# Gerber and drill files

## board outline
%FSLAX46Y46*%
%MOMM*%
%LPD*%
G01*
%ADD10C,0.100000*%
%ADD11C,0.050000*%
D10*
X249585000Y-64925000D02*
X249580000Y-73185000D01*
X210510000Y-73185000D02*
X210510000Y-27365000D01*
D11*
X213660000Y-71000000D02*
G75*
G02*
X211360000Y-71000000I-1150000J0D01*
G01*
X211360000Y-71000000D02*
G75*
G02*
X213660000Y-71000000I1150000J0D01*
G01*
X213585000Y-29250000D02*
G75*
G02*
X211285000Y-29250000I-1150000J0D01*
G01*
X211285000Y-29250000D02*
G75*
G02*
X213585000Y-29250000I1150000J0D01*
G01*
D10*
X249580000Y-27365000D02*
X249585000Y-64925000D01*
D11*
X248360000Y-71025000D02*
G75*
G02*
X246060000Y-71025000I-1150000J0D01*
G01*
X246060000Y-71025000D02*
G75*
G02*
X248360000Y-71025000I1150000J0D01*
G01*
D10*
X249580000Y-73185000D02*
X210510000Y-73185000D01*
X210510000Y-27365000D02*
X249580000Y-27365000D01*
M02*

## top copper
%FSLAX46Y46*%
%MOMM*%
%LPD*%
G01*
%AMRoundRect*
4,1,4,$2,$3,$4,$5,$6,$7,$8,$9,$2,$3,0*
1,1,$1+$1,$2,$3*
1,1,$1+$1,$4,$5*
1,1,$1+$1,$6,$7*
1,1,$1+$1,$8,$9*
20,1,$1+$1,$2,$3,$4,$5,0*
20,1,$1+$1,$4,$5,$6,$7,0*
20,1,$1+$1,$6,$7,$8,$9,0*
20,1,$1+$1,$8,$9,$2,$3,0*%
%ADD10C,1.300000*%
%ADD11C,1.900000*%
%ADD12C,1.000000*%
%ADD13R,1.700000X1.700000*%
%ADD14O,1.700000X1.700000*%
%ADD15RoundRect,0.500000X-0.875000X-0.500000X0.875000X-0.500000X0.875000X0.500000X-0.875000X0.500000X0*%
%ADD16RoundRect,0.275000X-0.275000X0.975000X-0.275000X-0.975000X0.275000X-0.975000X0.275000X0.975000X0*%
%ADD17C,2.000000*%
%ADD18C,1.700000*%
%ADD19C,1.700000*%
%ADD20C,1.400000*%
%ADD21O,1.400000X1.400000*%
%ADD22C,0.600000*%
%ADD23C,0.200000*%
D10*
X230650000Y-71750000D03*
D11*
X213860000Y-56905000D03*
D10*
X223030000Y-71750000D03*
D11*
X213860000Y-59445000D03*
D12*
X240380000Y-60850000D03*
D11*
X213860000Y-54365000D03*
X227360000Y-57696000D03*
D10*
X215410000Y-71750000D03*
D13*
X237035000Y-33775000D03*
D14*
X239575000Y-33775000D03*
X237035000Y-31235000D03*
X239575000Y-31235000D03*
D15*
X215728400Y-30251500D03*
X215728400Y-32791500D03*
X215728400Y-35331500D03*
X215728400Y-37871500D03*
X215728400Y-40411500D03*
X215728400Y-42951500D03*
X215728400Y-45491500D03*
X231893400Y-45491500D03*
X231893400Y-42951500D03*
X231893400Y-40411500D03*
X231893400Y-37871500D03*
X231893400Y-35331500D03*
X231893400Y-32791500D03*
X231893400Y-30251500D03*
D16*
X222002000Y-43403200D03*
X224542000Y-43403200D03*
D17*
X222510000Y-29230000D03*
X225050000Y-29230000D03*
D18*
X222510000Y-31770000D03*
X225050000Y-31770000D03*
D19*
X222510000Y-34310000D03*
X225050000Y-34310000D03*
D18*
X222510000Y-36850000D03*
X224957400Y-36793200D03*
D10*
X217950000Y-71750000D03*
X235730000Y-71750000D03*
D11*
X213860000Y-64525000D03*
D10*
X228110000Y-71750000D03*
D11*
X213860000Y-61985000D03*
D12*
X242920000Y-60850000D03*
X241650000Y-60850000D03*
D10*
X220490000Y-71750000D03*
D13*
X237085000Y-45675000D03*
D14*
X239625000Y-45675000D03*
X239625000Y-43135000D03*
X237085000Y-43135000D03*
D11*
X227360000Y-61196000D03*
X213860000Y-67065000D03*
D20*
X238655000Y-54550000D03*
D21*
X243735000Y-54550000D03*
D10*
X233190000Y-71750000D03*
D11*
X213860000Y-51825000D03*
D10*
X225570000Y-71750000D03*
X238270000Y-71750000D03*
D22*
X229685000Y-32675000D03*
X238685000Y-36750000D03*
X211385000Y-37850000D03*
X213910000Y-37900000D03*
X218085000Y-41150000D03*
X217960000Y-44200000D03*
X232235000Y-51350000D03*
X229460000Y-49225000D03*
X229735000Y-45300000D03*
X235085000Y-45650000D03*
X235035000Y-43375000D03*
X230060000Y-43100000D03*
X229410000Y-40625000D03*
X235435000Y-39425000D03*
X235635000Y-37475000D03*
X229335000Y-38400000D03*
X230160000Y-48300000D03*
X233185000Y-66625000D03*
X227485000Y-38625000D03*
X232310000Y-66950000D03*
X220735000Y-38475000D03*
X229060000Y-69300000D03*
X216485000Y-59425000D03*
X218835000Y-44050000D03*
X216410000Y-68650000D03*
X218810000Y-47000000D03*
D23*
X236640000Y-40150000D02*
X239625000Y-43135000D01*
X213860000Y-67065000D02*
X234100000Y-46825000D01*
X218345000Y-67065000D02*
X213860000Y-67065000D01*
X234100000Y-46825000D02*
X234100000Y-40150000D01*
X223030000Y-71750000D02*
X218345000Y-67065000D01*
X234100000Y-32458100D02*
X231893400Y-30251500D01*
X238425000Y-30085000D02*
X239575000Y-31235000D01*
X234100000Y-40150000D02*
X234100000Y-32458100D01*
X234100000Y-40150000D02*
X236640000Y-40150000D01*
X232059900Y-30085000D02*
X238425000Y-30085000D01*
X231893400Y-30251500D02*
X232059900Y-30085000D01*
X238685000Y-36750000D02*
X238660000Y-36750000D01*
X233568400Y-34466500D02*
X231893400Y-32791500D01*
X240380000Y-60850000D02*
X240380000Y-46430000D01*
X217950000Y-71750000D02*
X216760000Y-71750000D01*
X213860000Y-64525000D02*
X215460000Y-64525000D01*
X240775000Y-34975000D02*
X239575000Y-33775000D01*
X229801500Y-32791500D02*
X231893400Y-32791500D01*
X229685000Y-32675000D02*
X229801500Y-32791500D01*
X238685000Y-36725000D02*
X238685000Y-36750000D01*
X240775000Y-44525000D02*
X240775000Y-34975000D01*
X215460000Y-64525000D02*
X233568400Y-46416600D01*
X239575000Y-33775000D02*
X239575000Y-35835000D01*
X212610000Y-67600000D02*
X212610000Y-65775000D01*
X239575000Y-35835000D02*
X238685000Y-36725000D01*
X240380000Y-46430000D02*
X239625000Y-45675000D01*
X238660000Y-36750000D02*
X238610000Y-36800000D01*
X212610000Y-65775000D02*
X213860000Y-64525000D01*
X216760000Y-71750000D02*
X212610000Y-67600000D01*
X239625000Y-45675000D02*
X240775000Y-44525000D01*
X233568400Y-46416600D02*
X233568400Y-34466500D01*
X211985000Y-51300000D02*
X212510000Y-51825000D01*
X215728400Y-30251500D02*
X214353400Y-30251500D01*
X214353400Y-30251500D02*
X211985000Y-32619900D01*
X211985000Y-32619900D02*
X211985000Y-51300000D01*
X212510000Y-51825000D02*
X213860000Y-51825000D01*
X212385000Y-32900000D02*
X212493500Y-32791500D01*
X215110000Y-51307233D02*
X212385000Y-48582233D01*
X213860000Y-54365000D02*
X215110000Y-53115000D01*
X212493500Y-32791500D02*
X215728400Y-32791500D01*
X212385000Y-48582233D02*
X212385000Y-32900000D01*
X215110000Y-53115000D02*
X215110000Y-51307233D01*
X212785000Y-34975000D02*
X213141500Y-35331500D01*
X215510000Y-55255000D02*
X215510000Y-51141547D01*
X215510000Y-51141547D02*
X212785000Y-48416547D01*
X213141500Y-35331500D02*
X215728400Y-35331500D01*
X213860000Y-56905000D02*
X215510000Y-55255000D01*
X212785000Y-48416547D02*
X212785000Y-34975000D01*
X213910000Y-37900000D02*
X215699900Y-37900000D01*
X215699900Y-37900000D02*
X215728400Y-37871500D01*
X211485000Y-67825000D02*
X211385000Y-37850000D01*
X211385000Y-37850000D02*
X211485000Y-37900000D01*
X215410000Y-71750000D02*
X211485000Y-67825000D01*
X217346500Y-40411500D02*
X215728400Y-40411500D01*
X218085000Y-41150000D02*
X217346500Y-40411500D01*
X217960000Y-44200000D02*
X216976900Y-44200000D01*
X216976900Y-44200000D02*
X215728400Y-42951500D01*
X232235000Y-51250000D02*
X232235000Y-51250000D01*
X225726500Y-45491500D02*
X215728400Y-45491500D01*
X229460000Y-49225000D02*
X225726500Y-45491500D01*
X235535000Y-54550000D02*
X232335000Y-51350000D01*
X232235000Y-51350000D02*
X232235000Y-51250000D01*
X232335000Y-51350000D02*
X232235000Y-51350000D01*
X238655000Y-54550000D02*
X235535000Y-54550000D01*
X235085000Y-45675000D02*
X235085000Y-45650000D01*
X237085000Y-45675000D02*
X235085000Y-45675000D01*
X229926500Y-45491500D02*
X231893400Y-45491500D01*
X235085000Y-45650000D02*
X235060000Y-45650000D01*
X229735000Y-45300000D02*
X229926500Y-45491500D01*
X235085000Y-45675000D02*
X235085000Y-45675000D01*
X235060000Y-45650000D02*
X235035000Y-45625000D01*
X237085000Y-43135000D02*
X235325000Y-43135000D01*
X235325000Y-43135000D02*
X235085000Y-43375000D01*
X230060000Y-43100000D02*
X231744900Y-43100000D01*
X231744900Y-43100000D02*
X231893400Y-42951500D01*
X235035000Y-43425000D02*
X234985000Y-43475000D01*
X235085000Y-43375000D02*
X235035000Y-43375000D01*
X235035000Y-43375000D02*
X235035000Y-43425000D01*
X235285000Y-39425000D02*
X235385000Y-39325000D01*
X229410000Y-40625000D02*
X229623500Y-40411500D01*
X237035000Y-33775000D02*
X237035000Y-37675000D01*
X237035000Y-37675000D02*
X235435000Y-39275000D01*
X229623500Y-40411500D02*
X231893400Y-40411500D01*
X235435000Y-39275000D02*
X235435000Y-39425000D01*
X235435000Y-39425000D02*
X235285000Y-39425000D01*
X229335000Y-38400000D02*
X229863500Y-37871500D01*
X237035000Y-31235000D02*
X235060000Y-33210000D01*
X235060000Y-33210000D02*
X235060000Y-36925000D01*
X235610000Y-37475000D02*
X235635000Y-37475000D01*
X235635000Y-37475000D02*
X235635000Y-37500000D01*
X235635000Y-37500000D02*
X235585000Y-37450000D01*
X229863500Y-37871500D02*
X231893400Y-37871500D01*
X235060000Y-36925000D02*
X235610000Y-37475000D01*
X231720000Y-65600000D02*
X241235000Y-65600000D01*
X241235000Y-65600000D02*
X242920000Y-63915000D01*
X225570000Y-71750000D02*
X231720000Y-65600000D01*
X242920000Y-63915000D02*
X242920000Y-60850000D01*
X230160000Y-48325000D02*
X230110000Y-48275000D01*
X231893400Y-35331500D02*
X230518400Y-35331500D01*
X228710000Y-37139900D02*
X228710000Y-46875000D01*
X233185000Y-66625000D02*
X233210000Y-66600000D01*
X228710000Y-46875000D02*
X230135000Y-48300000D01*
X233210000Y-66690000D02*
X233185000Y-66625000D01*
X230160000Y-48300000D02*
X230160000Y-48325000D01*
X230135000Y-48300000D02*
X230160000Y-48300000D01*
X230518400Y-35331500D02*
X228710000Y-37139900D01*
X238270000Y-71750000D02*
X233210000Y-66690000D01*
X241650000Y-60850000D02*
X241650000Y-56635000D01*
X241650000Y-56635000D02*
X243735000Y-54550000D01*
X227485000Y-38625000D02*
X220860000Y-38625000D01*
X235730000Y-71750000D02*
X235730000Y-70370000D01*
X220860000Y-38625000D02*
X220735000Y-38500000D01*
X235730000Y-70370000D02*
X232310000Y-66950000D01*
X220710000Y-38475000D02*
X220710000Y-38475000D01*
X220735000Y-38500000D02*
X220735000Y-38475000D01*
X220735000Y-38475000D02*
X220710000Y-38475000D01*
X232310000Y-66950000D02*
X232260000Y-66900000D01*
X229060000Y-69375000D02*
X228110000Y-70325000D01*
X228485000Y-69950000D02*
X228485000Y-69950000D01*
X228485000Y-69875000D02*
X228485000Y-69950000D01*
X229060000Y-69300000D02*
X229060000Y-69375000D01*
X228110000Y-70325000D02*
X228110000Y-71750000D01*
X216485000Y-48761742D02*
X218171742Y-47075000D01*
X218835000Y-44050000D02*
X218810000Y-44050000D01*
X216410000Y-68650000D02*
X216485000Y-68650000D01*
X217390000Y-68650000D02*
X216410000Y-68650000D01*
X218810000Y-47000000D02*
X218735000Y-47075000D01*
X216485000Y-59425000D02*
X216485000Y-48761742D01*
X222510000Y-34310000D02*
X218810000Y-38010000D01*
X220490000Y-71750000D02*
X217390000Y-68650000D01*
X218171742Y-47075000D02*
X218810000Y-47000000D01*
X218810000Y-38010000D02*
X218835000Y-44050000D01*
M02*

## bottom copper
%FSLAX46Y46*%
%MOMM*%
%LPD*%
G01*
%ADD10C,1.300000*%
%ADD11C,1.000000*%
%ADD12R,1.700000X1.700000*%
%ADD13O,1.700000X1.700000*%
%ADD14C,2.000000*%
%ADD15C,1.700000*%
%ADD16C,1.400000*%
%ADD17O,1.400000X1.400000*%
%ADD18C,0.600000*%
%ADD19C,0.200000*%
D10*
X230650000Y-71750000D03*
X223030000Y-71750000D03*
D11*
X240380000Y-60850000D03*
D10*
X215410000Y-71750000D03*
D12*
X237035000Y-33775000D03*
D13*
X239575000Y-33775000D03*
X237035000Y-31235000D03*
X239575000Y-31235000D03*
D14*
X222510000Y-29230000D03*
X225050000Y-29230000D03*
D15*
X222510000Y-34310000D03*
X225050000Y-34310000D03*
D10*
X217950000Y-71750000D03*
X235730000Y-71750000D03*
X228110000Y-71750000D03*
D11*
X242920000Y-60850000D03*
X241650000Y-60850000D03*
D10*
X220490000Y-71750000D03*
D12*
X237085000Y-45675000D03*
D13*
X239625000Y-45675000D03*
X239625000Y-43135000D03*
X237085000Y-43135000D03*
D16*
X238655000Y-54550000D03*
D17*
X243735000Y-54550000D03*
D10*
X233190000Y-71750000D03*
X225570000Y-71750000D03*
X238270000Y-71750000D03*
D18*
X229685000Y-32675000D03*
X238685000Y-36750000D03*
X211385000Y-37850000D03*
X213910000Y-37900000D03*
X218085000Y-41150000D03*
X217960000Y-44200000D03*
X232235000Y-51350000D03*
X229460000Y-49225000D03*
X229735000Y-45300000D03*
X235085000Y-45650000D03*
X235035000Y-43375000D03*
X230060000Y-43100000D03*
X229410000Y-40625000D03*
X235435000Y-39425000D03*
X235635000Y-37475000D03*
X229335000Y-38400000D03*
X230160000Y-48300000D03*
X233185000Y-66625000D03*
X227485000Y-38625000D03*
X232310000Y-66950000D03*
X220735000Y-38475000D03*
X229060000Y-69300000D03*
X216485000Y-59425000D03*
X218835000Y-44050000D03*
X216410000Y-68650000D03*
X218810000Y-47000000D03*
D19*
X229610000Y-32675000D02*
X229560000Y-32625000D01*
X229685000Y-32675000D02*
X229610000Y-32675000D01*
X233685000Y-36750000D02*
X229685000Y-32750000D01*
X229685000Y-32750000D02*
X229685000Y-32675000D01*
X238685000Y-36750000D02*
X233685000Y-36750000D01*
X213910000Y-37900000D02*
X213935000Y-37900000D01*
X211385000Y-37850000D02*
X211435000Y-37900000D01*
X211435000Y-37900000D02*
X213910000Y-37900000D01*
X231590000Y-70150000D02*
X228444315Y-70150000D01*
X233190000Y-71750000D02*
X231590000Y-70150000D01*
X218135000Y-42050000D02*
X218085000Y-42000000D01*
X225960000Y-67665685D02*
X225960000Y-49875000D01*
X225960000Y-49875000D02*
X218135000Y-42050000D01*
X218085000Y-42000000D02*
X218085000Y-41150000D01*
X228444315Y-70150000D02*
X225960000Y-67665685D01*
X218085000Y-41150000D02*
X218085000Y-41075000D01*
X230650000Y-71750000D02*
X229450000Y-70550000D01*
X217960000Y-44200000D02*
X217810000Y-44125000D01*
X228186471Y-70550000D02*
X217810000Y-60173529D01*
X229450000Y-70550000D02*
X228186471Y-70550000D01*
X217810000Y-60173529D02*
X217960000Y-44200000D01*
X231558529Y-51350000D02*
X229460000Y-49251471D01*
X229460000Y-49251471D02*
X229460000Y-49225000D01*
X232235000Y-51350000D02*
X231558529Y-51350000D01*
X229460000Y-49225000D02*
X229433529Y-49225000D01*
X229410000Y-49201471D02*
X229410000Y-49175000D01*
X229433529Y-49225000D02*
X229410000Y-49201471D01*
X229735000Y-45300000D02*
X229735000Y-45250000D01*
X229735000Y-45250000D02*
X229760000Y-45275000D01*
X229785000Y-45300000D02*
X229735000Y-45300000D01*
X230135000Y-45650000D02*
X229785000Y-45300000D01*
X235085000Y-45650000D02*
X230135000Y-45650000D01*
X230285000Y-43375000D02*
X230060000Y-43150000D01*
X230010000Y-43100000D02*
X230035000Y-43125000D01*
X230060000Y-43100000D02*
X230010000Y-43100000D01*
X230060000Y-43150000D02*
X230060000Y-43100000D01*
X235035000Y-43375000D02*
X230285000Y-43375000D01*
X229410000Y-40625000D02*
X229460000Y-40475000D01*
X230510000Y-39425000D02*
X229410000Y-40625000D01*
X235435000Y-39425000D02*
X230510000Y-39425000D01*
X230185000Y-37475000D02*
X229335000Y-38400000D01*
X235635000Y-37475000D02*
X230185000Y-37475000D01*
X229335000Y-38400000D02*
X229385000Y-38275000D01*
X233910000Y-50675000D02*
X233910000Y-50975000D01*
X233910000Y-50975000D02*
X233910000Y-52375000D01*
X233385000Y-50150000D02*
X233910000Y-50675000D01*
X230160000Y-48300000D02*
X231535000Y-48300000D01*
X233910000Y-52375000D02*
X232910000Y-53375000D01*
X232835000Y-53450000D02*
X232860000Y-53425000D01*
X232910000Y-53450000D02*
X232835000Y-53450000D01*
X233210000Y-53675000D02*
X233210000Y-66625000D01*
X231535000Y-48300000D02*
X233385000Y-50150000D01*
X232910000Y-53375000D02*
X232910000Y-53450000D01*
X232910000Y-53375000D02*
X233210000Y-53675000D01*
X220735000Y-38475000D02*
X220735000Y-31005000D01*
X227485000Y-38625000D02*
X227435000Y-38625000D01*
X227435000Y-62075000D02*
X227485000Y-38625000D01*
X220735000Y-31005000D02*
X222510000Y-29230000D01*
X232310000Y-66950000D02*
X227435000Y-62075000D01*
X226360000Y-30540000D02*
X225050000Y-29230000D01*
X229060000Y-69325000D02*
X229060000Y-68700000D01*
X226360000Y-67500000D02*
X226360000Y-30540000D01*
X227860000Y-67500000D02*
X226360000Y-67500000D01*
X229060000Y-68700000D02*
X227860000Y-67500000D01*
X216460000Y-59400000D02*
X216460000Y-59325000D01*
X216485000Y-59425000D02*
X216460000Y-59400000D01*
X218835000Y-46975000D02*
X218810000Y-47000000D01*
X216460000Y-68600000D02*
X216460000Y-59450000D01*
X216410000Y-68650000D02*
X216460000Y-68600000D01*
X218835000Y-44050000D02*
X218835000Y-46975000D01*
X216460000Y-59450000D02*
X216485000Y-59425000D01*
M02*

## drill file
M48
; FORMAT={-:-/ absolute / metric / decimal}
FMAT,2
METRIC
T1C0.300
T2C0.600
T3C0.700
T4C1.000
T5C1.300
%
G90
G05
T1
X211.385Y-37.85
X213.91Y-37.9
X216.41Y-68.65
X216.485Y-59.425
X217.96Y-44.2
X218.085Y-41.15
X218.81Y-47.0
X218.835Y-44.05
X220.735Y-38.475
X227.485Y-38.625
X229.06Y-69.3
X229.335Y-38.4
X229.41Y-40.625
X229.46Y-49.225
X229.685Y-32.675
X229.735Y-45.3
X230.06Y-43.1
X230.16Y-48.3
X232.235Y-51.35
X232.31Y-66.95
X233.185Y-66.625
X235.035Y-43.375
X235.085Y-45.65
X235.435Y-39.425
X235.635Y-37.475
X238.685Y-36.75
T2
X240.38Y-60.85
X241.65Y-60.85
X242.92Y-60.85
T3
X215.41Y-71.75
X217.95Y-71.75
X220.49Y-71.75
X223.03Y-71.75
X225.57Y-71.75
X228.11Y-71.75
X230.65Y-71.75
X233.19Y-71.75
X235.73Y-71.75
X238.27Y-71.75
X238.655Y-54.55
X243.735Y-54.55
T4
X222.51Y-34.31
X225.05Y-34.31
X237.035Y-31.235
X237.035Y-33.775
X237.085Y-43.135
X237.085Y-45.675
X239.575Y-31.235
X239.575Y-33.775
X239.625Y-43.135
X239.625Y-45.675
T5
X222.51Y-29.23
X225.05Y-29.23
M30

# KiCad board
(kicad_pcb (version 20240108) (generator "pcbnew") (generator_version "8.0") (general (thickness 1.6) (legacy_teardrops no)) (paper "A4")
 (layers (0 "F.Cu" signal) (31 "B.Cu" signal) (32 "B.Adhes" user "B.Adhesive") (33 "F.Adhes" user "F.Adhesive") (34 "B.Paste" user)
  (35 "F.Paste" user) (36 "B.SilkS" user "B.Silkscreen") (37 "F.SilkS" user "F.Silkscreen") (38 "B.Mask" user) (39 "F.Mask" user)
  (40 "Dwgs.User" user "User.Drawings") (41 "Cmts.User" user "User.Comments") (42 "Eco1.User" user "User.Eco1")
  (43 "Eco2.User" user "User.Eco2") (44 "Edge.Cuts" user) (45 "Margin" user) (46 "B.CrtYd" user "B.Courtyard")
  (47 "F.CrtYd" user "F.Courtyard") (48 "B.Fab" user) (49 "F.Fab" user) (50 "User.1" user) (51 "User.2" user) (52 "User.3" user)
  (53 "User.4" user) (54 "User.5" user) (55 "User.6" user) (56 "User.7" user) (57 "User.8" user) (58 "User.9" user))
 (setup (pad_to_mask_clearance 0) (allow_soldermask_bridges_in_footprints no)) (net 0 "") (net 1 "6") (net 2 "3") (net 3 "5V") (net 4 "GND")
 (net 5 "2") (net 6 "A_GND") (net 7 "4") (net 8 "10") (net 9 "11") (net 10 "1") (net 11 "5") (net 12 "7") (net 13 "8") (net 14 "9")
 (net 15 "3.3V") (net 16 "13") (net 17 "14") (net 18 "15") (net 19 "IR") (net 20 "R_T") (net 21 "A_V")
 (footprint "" (layer "F.Cu") (at 230.65 71.75)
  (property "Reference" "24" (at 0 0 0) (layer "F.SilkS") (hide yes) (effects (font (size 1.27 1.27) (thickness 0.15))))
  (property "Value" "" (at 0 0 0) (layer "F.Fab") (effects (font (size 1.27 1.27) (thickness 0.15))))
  (pad "" thru_hole circle (at 0 0 180) (size 1.3 1.3) (drill 0.7) (layers "*.Cu" "*.Mask") (remove_unused_layers no) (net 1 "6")))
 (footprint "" (layer "F.Cu") (at 228.21 55.536 90)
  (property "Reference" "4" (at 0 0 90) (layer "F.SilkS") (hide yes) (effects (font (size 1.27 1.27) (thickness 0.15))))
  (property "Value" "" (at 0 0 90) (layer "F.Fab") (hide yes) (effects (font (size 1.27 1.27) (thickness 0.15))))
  (pad "6" smd circle (at -1.369 -14.35 270) (size 1.9 1.9) (layers "F.Cu" "F.Mask") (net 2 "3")))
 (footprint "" (layer "F.Cu") (at 223.03 71.75)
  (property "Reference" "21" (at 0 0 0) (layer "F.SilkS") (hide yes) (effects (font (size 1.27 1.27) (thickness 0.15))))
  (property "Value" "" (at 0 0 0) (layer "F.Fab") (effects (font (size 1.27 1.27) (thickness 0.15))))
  (pad "" thru_hole circle (at 0 0 180) (size 1.3 1.3) (drill 0.7) (layers "*.Cu" "*.Mask") (remove_unused_layers no) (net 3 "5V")))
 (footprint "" (layer "F.Cu") (at 228.21 58.076 90)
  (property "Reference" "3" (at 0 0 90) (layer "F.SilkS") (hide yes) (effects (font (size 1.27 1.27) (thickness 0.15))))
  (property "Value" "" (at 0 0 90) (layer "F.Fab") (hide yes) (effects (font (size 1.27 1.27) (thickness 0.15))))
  (pad "6" smd circle (at -1.369 -14.35 270) (size 1.9 1.9) (layers "F.Cu" "F.Mask")))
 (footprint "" (layer "F.Cu") (at 240.38 60.85)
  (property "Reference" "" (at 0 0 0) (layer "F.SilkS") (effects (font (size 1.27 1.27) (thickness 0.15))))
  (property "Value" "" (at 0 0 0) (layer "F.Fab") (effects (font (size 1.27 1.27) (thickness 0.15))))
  (pad "" thru_hole circle (at 0 0 180) (size 1 1) (drill 0.6) (layers "*.Cu" "*.Mask") (remove_unused_layers no) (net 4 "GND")))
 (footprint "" (layer "F.Cu") (at 228.21 52.996 90)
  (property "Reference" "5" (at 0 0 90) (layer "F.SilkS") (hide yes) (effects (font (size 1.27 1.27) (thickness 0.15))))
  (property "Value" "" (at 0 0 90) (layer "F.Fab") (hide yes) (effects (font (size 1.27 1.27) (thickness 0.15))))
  (pad "6" smd circle (at -1.369 -14.35 270) (size 1.9 1.9) (layers "F.Cu" "F.Mask") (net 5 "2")))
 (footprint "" (layer "F.Cu") (at 240.535 56.877 90)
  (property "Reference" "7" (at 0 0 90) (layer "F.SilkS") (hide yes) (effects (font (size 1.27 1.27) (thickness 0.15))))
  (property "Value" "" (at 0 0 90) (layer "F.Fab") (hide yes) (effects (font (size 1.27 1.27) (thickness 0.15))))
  (pad "6" smd circle (at -0.819 -13.175 270) (size 1.9 1.9) (layers "F.Cu" "F.Mask") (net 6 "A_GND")))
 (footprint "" (layer "F.Cu") (at 215.41 71.75)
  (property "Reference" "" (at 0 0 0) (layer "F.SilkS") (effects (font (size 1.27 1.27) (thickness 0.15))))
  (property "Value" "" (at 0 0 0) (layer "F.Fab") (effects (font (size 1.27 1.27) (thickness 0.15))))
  (pad "" thru_hole circle (at 0 0 180) (size 1.3 1.3) (drill 0.7) (layers "*.Cu" "*.Mask") (remove_unused_layers no) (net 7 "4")))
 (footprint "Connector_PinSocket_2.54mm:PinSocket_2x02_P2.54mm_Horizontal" (layer "F.Cu") (at 237.035 33.775 180)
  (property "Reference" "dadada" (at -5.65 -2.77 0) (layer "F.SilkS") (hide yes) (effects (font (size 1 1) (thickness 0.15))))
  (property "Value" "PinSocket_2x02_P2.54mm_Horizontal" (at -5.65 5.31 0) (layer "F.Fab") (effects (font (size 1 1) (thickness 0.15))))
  (pad "1" thru_hole rect (at 0 0 180) (size 1.7 1.7) (drill 1) (layers "*.Cu" "*.Mask") (remove_unused_layers no) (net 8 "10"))
  (pad "2" thru_hole oval (at -2.54 0 180) (size 1.7 1.7) (drill 1) (layers "*.Cu" "*.Mask") (remove_unused_layers no) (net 4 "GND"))
  (pad "3" thru_hole oval (at 0 2.54 180) (size 1.7 1.7) (drill 1) (layers "*.Cu" "*.Mask") (remove_unused_layers no) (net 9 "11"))
  (pad "4" thru_hole oval (at -2.54 2.54 180) (size 1.7 1.7) (drill 1) (layers "*.Cu" "*.Mask") (remove_unused_layers no) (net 3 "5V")))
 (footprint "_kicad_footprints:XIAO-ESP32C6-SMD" (layer "F.Cu") (at 224.01 37.85)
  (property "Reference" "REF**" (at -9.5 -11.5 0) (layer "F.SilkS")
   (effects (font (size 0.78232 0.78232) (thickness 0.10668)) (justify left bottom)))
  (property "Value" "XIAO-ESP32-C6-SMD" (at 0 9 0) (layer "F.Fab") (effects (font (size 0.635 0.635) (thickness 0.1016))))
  (pad "1" smd roundrect (at -8.2816 -7.5985) (size 2.75 2) (layers "F.Cu" "F.Paste" "F.Mask") (roundrect_rratio 0.25) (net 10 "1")
   (solder_mask_margin 0.0508) (thermal_bridge_angle 45))
  (pad "2" smd roundrect (at -8.2816 -5.0585) (size 2.75 2) (layers "F.Cu" "F.Paste" "F.Mask") (roundrect_rratio 0.25) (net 5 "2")
   (solder_mask_margin 0.0508) (thermal_bridge_angle 45))
  (pad "3" smd roundrect (at -8.2816 -2.5185) (size 2.75 2) (layers "F.Cu" "F.Paste" "F.Mask") (roundrect_rratio 0.25) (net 2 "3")
   (solder_mask_margin 0.0508) (thermal_bridge_angle 45))
  (pad "4" smd roundrect (at -8.2816 0.0215) (size 2.75 2) (layers "F.Cu" "F.Paste" "F.Mask") (roundrect_rratio 0.25) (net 7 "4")
   (solder_mask_margin 0.0508) (thermal_bridge_angle 45))
  (pad "5" smd roundrect (at -8.2816 2.5615) (size 2.75 2) (layers "F.Cu" "F.Paste" "F.Mask") (roundrect_rratio 0.25) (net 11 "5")
   (solder_mask_margin 0.0508) (thermal_bridge_angle 45))
  (pad "6" smd roundrect (at -8.2816 5.1015) (size 2.75 2) (layers "F.Cu" "F.Paste" "F.Mask") (roundrect_rratio 0.25) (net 1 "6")
   (solder_mask_margin 0.0508) (thermal_bridge_angle 45))
  (pad "7" smd roundrect (at -8.2816 7.6415) (size 2.75 2) (layers "F.Cu" "F.Paste" "F.Mask") (roundrect_rratio 0.25) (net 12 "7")
   (solder_mask_margin 0.0508) (thermal_bridge_angle 45))
  (pad "8" smd roundrect (at 7.8834 7.6415) (size 2.75 2) (layers "F.Cu" "F.Paste" "F.Mask") (roundrect_rratio 0.25) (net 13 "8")
   (solder_mask_margin 0.0508) (thermal_bridge_angle 45))
  (pad "9" smd roundrect (at 7.8834 5.1015) (size 2.75 2) (layers "F.Cu" "F.Paste" "F.Mask") (roundrect_rratio 0.25) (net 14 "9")
   (solder_mask_margin 0.0508) (thermal_bridge_angle 45))
  (pad "10" smd roundrect (at 7.8834 2.5615) (size 2.75 2) (layers "F.Cu" "F.Paste" "F.Mask") (roundrect_rratio 0.25) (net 8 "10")
   (solder_mask_margin 0.0508) (thermal_bridge_angle 45))
  (pad "11" smd roundrect (at 7.8834 0.0215) (size 2.75 2) (layers "F.Cu" "F.Paste" "F.Mask") (roundrect_rratio 0.25) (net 9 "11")
   (solder_mask_margin 0.0508) (thermal_bridge_angle 45))
  (pad "12" smd roundrect (at 7.8834 -2.5185) (size 2.75 2) (layers "F.Cu" "F.Paste" "F.Mask") (roundrect_rratio 0.25) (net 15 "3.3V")
   (solder_mask_margin 0.0508) (thermal_bridge_angle 45))
  (pad "13" smd roundrect (at 7.8834 -5.0585) (size 2.75 2) (layers "F.Cu" "F.Paste" "F.Mask") (roundrect_rratio 0.25) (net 4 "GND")
   (solder_mask_margin 0.0508) (thermal_bridge_angle 45))
  (pad "14" smd roundrect (at 7.8834 -7.5985) (size 2.75 2) (layers "F.Cu" "F.Paste" "F.Mask") (roundrect_rratio 0.25) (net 3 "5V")
   (solder_mask_margin 0.0508) (thermal_bridge_angle 45))
  (pad "15" smd roundrect (at -2.008 5.5532 270) (size 2.5 1.1) (layers "F.Cu" "F.Paste" "F.Mask") (roundrect_rratio 0.25)
   (solder_mask_margin 0.0508) (thermal_bridge_angle 45))
  (pad "16" smd roundrect (at 0.532 5.5532 270) (size 2.5 1.1) (layers "F.Cu" "F.Paste" "F.Mask") (roundrect_rratio 0.25)
   (solder_mask_margin 0.0508) (thermal_bridge_angle 45))
  (pad "17" thru_hole circle (at -1.5 -8.62) (size 2 2) (drill 1.3) (layers "*.Cu" "*.Mask") (remove_unused_layers no) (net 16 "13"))
  (pad "18" thru_hole circle (at 1.04 -8.62) (size 2 2) (drill 1.3) (layers "*.Cu" "*.Mask") (remove_unused_layers no) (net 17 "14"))
  (pad "19" smd circle (at -1.5 -6.08) (size 1.7 1.7) (layers "F.Cu" "F.Paste" "F.Mask"))
  (pad "20" smd circle (at 1.04 -6.08) (size 1.7 1.7) (layers "F.Cu" "F.Paste" "F.Mask"))
  (pad "21" thru_hole circle (at -1.5 -3.54) (size 1.7 1.7) (drill 1) (layers "*.Cu" "*.Mask") (remove_unused_layers no) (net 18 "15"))
  (pad "22" thru_hole circle (at 1.04 -3.54) (size 1.7 1.7) (drill 1) (layers "*.Cu" "*.Mask") (remove_unused_layers no))
  (pad "23" smd circle (at -1.5 -1) (size 1.7 1.7) (layers "F.Cu" "F.Paste" "F.Mask"))
  (pad "24" smd circle (at 0.9474 -1.0568) (size 1.7 1.7) (layers "F.Cu" "F.Paste" "F.Mask")))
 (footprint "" (layer "F.Cu") (at 217.95 71.75)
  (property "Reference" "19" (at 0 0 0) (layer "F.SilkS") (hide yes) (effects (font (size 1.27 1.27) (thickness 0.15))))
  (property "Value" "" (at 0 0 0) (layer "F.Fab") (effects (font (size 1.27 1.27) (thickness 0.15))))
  (pad "" thru_hole circle (at 0 0 180) (size 1.3 1.3) (drill 0.7) (layers "*.Cu" "*.Mask") (remove_unused_layers no) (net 4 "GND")))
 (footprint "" (layer "F.Cu") (at 235.73 71.75)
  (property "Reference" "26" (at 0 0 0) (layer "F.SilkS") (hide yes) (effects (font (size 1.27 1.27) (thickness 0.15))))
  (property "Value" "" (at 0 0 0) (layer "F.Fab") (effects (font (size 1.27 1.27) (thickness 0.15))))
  (pad "" thru_hole circle (at 0 0 180) (size 1.3 1.3) (drill 0.7) (layers "*.Cu" "*.Mask") (remove_unused_layers no) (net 16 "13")))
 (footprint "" (layer "F.Cu") (at 228.21 63.156 90)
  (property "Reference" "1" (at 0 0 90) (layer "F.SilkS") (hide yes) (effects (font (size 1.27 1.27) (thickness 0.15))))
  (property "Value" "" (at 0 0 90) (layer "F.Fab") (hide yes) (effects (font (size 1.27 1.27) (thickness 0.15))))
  (pad "6" smd circle (at -1.369 -14.35 270) (size 1.9 1.9) (layers "F.Cu" "F.Mask") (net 4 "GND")))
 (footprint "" (layer "F.Cu") (at 228.11 71.75)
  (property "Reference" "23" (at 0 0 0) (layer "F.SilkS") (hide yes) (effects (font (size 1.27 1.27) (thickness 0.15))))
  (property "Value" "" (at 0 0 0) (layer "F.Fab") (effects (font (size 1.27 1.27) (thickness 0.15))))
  (pad "" thru_hole circle (at 0 0 180) (size 1.3 1.3) (drill 0.7) (layers "*.Cu" "*.Mask") (remove_unused_layers no) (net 17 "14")))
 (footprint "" (layer "F.Cu") (at 228.21 60.616 90)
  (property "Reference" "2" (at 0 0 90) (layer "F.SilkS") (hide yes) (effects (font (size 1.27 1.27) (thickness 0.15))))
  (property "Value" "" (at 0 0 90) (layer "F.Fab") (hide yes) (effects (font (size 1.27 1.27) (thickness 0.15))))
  (pad "6" smd circle (at -1.369 -14.35 270) (size 1.9 1.9) (layers "F.Cu" "F.Mask")))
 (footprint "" (layer "F.Cu") (at 242.92 60.85)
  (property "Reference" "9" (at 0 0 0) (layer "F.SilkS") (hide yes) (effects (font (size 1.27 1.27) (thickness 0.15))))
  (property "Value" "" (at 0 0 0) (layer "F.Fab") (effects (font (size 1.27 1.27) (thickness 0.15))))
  (pad "" thru_hole circle (at 0 0 180) (size 1 1) (drill 0.6) (layers "*.Cu" "*.Mask") (remove_unused_layers no) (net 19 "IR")))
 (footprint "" (layer "F.Cu") (at 241.65 60.85)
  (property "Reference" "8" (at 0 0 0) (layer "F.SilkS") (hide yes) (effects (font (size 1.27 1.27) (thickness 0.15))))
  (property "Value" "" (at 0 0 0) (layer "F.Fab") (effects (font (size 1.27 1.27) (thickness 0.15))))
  (pad "" thru_hole circle (at 0 0 180) (size 1 1) (drill 0.6) (layers "*.Cu" "*.Mask") (remove_unused_layers no) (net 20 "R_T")))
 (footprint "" (layer "F.Cu") (at 220.49 71.75)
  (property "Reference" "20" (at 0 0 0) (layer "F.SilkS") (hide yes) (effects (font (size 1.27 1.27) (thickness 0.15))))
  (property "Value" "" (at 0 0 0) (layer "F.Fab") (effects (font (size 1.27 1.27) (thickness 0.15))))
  (pad "" thru_hole circle (at 0 0 180) (size 1.3 1.3) (drill 0.7) (layers "*.Cu" "*.Mask") (remove_unused_layers no) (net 18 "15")))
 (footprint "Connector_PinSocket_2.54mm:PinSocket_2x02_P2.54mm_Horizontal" (layer "F.Cu") (at 237.085 45.675 180)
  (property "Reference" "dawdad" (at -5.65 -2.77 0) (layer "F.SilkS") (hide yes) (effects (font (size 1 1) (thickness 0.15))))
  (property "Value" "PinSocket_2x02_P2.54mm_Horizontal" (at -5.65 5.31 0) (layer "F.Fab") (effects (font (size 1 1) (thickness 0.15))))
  (pad "1" thru_hole rect (at 0 0 180) (size 1.7 1.7) (drill 1) (layers "*.Cu" "*.Mask") (remove_unused_layers no) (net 13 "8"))
  (pad "2" thru_hole oval (at -2.54 0 180) (size 1.7 1.7) (drill 1) (layers "*.Cu" "*.Mask") (remove_unused_layers no) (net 4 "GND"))
  (pad "2" thru_hole oval (at -2.54 2.54 180) (size 1.7 1.7) (drill 1) (layers "*.Cu" "*.Mask") (remove_unused_layers no) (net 3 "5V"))
  (pad "eeeeee" thru_hole oval (at 0 2.54 180) (size 1.7 1.7) (drill 1) (layers "*.Cu" "*.Mask") (remove_unused_layers no) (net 14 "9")))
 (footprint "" (layer "F.Cu") (at 240.535 60.377 90)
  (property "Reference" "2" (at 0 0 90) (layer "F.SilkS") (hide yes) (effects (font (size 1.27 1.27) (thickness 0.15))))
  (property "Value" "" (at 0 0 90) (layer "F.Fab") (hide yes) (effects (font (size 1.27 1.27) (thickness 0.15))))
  (pad "6" smd circle (at -0.819 -13.175 270) (size 1.9 1.9) (layers "F.Cu" "F.Mask") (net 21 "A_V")))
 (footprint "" (layer "F.Cu") (at 228.21 65.696 90)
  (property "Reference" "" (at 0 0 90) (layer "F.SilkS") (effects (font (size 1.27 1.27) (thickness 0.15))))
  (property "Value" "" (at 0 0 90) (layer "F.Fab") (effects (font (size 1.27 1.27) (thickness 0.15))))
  (pad "6" smd circle (at -1.369 -14.35 270) (size 1.9 1.9) (layers "F.Cu" "F.Mask") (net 3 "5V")))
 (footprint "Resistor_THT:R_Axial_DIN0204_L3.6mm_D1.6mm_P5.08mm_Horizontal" (layer "F.Cu") (at 238.655 54.55)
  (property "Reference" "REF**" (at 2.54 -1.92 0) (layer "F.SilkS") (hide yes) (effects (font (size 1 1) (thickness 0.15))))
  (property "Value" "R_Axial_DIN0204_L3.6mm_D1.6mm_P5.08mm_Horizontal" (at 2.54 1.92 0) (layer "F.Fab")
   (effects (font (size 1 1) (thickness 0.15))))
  (pad "1" thru_hole circle (at 0 0) (size 1.4 1.4) (drill 0.7) (layers "*.Cu" "*.Mask") (remove_unused_layers no) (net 12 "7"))
  (pad "2" thru_hole oval (at 5.08 0) (size 1.4 1.4) (drill 0.7) (layers "*.Cu" "*.Mask") (remove_unused_layers no) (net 20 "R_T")))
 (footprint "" (layer "F.Cu") (at 233.19 71.75)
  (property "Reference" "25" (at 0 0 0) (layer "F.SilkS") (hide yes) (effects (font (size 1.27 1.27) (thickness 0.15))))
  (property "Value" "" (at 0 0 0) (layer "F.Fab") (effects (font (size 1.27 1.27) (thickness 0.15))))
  (pad "" thru_hole circle (at 0 0 180) (size 1.3 1.3) (drill 0.7) (layers "*.Cu" "*.Mask") (remove_unused_layers no) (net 11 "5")))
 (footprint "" (layer "F.Cu") (at 228.21 50.456 90)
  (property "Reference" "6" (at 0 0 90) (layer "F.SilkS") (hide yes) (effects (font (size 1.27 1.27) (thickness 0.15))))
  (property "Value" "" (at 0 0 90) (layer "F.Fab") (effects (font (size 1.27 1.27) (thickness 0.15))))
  (pad "6" smd circle (at -1.369 -14.35 270) (size 1.9 1.9) (layers "F.Cu" "F.Mask") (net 10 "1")))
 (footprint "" (layer "F.Cu") (at 225.57 71.75)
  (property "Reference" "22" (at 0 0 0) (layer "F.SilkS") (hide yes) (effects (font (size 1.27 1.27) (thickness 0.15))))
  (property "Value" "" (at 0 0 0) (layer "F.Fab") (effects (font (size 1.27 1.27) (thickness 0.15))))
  (pad "e" thru_hole circle (at 0 0 180) (size 1.3 1.3) (drill 0.7) (layers "*.Cu" "*.Mask") (remove_unused_layers no) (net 19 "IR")))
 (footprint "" (layer "F.Cu") (at 238.27 71.75)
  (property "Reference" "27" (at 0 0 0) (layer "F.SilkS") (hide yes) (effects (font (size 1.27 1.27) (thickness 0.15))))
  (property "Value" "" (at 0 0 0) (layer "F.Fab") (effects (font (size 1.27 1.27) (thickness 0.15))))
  (pad "" thru_hole circle (at 0 0 180) (size 1.3 1.3) (drill 0.7) (layers "*.Cu" "*.Mask") (remove_unused_layers no) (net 15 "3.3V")))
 (gr_line (start 249.585 64.925) (end 249.58 73.185) (stroke (width 0.1) (type default)) (layer "Edge.Cuts"))
 (gr_line (start 210.51 73.185) (end 210.51 27.365) (stroke (width 0.1) (type default)) (layer "Edge.Cuts"))
 (gr_circle (center 212.51 71) (end 213.66 71) (stroke (width 0.05) (type default)) (fill none) (layer "Edge.Cuts"))
 (gr_circle (center 212.435 29.25) (end 213.585 29.25) (stroke (width 0.05) (type default)) (fill none) (layer "Edge.Cuts"))
 (gr_line (start 249.58 27.365) (end 249.585 64.925) (stroke (width 0.1) (type default)) (layer "Edge.Cuts"))
 (gr_circle (center 247.21 71.025) (end 248.36 71.025) (stroke (width 0.05) (type default)) (fill none) (layer "Edge.Cuts"))
 (gr_line (start 249.58 73.185) (end 210.51 73.185) (stroke (width 0.1) (type default)) (layer "Edge.Cuts"))
 (gr_line (start 210.51 27.365) (end 249.58 27.365) (stroke (width 0.1) (type default)) (layer "Edge.Cuts"))
 (segment (start 236.64 40.15) (end 239.625 43.135) (width 0.2) (layer "F.Cu") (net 3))
 (segment (start 213.86 67.065) (end 234.1 46.825) (width 0.2) (layer "F.Cu") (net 3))
 (segment (start 218.345 67.065) (end 213.86 67.065) (width 0.2) (layer "F.Cu") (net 3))
 (segment (start 234.1 46.825) (end 234.1 40.15) (width 0.2) (layer "F.Cu") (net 3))
 (segment (start 223.03 71.75) (end 218.345 67.065) (width 0.2) (layer "F.Cu") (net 3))
 (segment (start 234.1 32.4581) (end 231.8934 30.2515) (width 0.2) (layer "F.Cu") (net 3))
 (segment (start 238.425 30.085) (end 239.575 31.235) (width 0.2) (layer "F.Cu") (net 3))
 (segment (start 234.1 40.15) (end 234.1 32.4581) (width 0.2) (layer "F.Cu") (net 3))
 (segment (start 234.1 40.15) (end 236.64 40.15) (width 0.2) (layer "F.Cu") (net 3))
 (segment (start 232.0599 30.085) (end 238.425 30.085) (width 0.2) (layer "F.Cu") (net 3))
 (segment (start 231.8934 30.2515) (end 232.0599 30.085) (width 0.2) (layer "F.Cu") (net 3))
 (segment (start 238.685 36.75) (end 238.66 36.75) (width 0.2) (layer "F.Cu") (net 4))
 (segment (start 233.5684 34.4665) (end 231.8934 32.7915) (width 0.2) (layer "F.Cu") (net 4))
 (segment (start 240.38 60.85) (end 240.38 46.43) (width 0.2) (layer "F.Cu") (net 4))
 (segment (start 217.95 71.75) (end 216.76 71.75) (width 0.2) (layer "F.Cu") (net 4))
 (segment (start 213.86 64.525) (end 215.46 64.525) (width 0.2) (layer "F.Cu") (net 4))
 (segment (start 240.775 34.975) (end 239.575 33.775) (width 0.2) (layer "F.Cu") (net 4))
 (segment (start 229.8015 32.7915) (end 231.8934 32.7915) (width 0.2) (layer "F.Cu") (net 4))
 (segment (start 229.685 32.675) (end 229.8015 32.7915) (width 0.2) (layer "F.Cu") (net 4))
 (segment (start 238.685 36.725) (end 238.685 36.75) (width 0.2) (layer "F.Cu") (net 4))
 (segment (start 240.775 44.525) (end 240.775 34.975) (width 0.2) (layer "F.Cu") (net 4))
 (segment (start 215.46 64.525) (end 233.5684 46.4166) (width 0.2) (layer "F.Cu") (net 4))
 (segment (start 239.575 33.775) (end 239.575 35.835) (width 0.2) (layer "F.Cu") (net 4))
 (segment (start 212.61 67.6) (end 212.61 65.775) (width 0.2) (layer "F.Cu") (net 4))
 (segment (start 239.575 35.835) (end 238.685 36.725) (width 0.2) (layer "F.Cu") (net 4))
 (segment (start 240.38 46.43) (end 239.625 45.675) (width 0.2) (layer "F.Cu") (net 4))
 (segment (start 238.66 36.75) (end 238.61 36.8) (width 0.2) (layer "F.Cu") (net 4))
 (segment (start 212.61 65.775) (end 213.86 64.525) (width 0.2) (layer "F.Cu") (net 4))
 (segment (start 216.76 71.75) (end 212.61 67.6) (width 0.2) (layer "F.Cu") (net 4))
 (segment (start 239.625 45.675) (end 240.775 44.525) (width 0.2) (layer "F.Cu") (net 4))
 (segment (start 233.5684 46.4166) (end 233.5684 34.4665) (width 0.2) (layer "F.Cu") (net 4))
 (via (at 229.685 32.675) (size 0.6) (drill 0.3) (layers "F.Cu" "B.Cu") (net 4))
 (via (at 238.685 36.75) (size 0.6) (drill 0.3) (layers "F.Cu" "B.Cu") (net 4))
 (segment (start 229.61 32.675) (end 229.56 32.625) (width 0.2) (layer "B.Cu") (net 4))
 (segment (start 229.685 32.675) (end 229.61 32.675) (width 0.2) (layer "B.Cu") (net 4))
 (segment (start 233.685 36.75) (end 229.685 32.75) (width 0.2) (layer "B.Cu") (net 4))
 (segment (start 229.685 32.75) (end 229.685 32.675) (width 0.2) (layer "B.Cu") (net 4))
 (segment (start 238.685 36.75) (end 233.685 36.75) (width 0.2) (layer "B.Cu") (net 4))
 (segment (start 211.985 51.3) (end 212.51 51.825) (width 0.2) (layer "F.Cu") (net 10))
 (segment (start 215.7284 30.2515) (end 214.3534 30.2515) (width 0.2) (layer "F.Cu") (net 10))
 (segment (start 214.3534 30.2515) (end 211.985 32.6199) (width 0.2) (layer "F.Cu") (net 10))
 (segment (start 211.985 32.6199) (end 211.985 51.3) (width 0.2) (layer "F.Cu") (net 10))
 (segment (start 212.51 51.825) (end 213.86 51.825) (width 0.2) (layer "F.Cu") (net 10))
 (segment (start 212.385 32.9) (end 212.4935 32.7915) (width 0.2) (layer "F.Cu") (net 5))
 (segment (start 215.11 51.307233) (end 212.385 48.582233) (width 0.2) (layer "F.Cu") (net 5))
 (segment (start 213.86 54.365) (end 215.11 53.115) (width 0.2) (layer "F.Cu") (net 5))
 (segment (start 212.4935 32.7915) (end 215.7284 32.7915) (width 0.2) (layer "F.Cu") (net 5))
 (segment (start 212.385 48.582233) (end 212.385 32.9) (width 0.2) (layer "F.Cu") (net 5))
 (segment (start 215.11 53.115) (end 215.11 51.307233) (width 0.2) (layer "F.Cu") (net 5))
 (segment (start 212.785 34.975) (end 213.1415 35.3315) (width 0.2) (layer "F.Cu") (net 2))
 (segment (start 215.51 55.255) (end 215.51 51.141547) (width 0.2) (layer "F.Cu") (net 2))
 (segment (start 215.51 51.141547) (end 212.785 48.416547) (width 0.2) (layer "F.Cu") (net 2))
 (segment (start 213.1415 35.3315) (end 215.7284 35.3315) (width 0.2) (layer "F.Cu") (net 2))
 (segment (start 213.86 56.905) (end 215.51 55.255) (width 0.2) (layer "F.Cu") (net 2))
 (segment (start 212.785 48.416547) (end 212.785 34.975) (width 0.2) (layer "F.Cu") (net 2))
 (segment (start 213.91 37.9) (end 215.6999 37.9) (width 0.2) (layer "F.Cu") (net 7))
 (segment (start 215.6999 37.9) (end 215.7284 37.8715) (width 0.2) (layer "F.Cu") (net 7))
 (segment (start 211.485 67.825) (end 211.385 37.85) (width 0.2) (layer "F.Cu") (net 7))
 (segment (start 211.385 37.85) (end 211.485 37.9) (width 0.2) (layer "F.Cu") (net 7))
 (segment (start 215.41 71.75) (end 211.485 67.825) (width 0.2) (layer "F.Cu") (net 7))
 (via (at 211.385 37.85) (size 0.6) (drill 0.3) (layers "F.Cu" "B.Cu") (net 7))
 (via (at 213.91 37.9) (size 0.6) (drill 0.3) (layers "F.Cu" "B.Cu") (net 7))
 (segment (start 213.91 37.9) (end 213.935 37.9) (width 0.2) (layer "B.Cu") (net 7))
 (segment (start 211.385 37.85) (end 211.435 37.9) (width 0.2) (layer "B.Cu") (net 7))
 (segment (start 211.435 37.9) (end 213.91 37.9) (width 0.2) (layer "B.Cu") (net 7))
 (segment (start 217.3465 40.4115) (end 215.7284 40.4115) (width 0.2) (layer "F.Cu") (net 11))
 (segment (start 218.085 41.15) (end 217.3465 40.4115) (width 0.2) (layer "F.Cu") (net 11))
 (via (at 218.085 41.15) (size 0.6) (drill 0.3) (layers "F.Cu" "B.Cu") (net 11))
 (segment (start 231.59 70.15) (end 228.444315 70.15) (width 0.2) (layer "B.Cu") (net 11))
 (segment (start 233.19 71.75) (end 231.59 70.15) (width 0.2) (layer "B.Cu") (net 11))
 (segment (start 218.135 42.05) (end 218.085 42) (width 0.2) (layer "B.Cu") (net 11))
 (segment (start 225.96 67.665685) (end 225.96 49.875) (width 0.2) (layer "B.Cu") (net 11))
 (segment (start 225.96 49.875) (end 218.135 42.05) (width 0.2) (layer "B.Cu") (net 11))
 (segment (start 218.085 42) (end 218.085 41.15) (width 0.2) (layer "B.Cu") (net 11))
 (segment (start 228.444315 70.15) (end 225.96 67.665685) (width 0.2) (layer "B.Cu") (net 11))
 (segment (start 218.085 41.15) (end 218.085 41.075) (width 0.2) (layer "B.Cu") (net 11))
 (segment (start 217.96 44.2) (end 216.9769 44.2) (width 0.2) (layer "F.Cu") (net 1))
 (segment (start 216.9769 44.2) (end 215.7284 42.9515) (width 0.2) (layer "F.Cu") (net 1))
 (via (at 217.96 44.2) (size 0.6) (drill 0.3) (layers "F.Cu" "B.Cu") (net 1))
 (segment (start 230.65 71.75) (end 229.45 70.55) (width 0.2) (layer "B.Cu") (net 1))
 (segment (start 217.96 44.2) (end 217.81 44.125) (width 0.2) (layer "B.Cu") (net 1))
 (segment (start 228.186471 70.55) (end 217.81 60.173529) (width 0.2) (layer "B.Cu") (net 1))
 (segment (start 229.45 70.55) (end 228.186471 70.55) (width 0.2) (layer "B.Cu") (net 1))
 (segment (start 217.81 60.173529) (end 217.96 44.2) (width 0.2) (layer "B.Cu") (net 1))
 (segment (start 232.235 51.25) (end 232.235 51.25) (width 0.2) (layer "F.Cu") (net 12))
 (segment (start 225.7265 45.4915) (end 215.7284 45.4915) (width 0.2) (layer "F.Cu") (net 12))
 (segment (start 229.46 49.225) (end 225.7265 45.4915) (width 0.2) (layer "F.Cu") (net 12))
 (segment (start 235.535 54.55) (end 232.335 51.35) (width 0.2) (layer "F.Cu") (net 12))
 (segment (start 232.235 51.35) (end 232.235 51.25) (width 0.2) (layer "F.Cu") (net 12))
 (segment (start 232.335 51.35) (end 232.235 51.35) (width 0.2) (layer "F.Cu") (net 12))
 (segment (start 238.655 54.55) (end 235.535 54.55) (width 0.2) (layer "F.Cu") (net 12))
 (via (at 232.235 51.35) (size 0.6) (drill 0.3) (layers "F.Cu" "B.Cu") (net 12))
 (via (at 229.46 49.225) (size 0.6) (drill 0.3) (layers "F.Cu" "B.Cu") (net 12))
 (segment (start 231.558529 51.35) (end 229.46 49.251471) (width 0.2) (layer "B.Cu") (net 12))
 (segment (start 229.46 49.251471) (end 229.46 49.225) (width 0.2) (layer "B.Cu") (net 12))
 (segment (start 232.235 51.35) (end 231.558529 51.35) (width 0.2) (layer "B.Cu") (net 12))
 (segment (start 229.46 49.225) (end 229.433529 49.225) (width 0.2) (layer "B.Cu") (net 12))
 (segment (start 229.41 49.201471) (end 229.41 49.175) (width 0.2) (layer "B.Cu") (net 12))
 (segment (start 229.433529 49.225) (end 229.41 49.201471) (width 0.2) (layer "B.Cu") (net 12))
 (segment (start 235.085 45.675) (end 235.085 45.65) (width 0.2) (layer "F.Cu") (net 13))
 (segment (start 237.085 45.675) (end 235.085 45.675) (width 0.2) (layer "F.Cu") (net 13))
 (segment (start 229.9265 45.4915) (end 231.8934 45.4915) (width 0.2) (layer "F.Cu") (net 13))
 (segment (start 235.085 45.65) (end 235.06 45.65) (width 0.2) (layer "F.Cu") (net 13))
 (segment (start 229.735 45.3) (end 229.9265 45.4915) (width 0.2) (layer "F.Cu") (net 13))
 (segment (start 235.085 45.675) (end 235.085 45.675) (width 0.2) (layer "F.Cu") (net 13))
 (segment (start 235.06 45.65) (end 235.035 45.625) (width 0.2) (layer "F.Cu") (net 13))
 (via (at 229.735 45.3) (size 0.6) (drill 0.3) (layers "F.Cu" "B.Cu") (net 13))
 (via (at 235.085 45.65) (size 0.6) (drill 0.3) (layers "F.Cu" "B.Cu") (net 13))
 (segment (start 229.735 45.3) (end 229.735 45.25) (width 0.2) (layer "B.Cu") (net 13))
 (segment (start 229.735 45.25) (end 229.76 45.275) (width 0.2) (layer "B.Cu") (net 13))
 (segment (start 229.785 45.3) (end 229.735 45.3) (width 0.2) (layer "B.Cu") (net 13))
 (segment (start 230.135 45.65) (end 229.785 45.3) (width 0.2) (layer "B.Cu") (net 13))
 (segment (start 235.085 45.65) (end 230.135 45.65) (width 0.2) (layer "B.Cu") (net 13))
 (segment (start 237.085 43.135) (end 235.325 43.135) (width 0.2) (layer "F.Cu") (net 14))
 (segment (start 235.325 43.135) (end 235.085 43.375) (width 0.2) (layer "F.Cu") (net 14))
 (segment (start 230.06 43.1) (end 231.7449 43.1) (width 0.2) (layer "F.Cu") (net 14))
 (segment (start 231.7449 43.1) (end 231.8934 42.9515) (width 0.2) (layer "F.Cu") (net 14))
 (segment (start 235.035 43.425) (end 234.985 43.475) (width 0.2) (layer "F.Cu") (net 14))
 (segment (start 235.085 43.375) (end 235.035 43.375) (width 0.2) (layer "F.Cu") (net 14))
 (segment (start 235.035 43.375) (end 235.035 43.425) (width 0.2) (layer "F.Cu") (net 14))
 (via (at 235.035 43.375) (size 0.6) (drill 0.3) (layers "F.Cu" "B.Cu") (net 14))
 (via (at 230.06 43.1) (size 0.6) (drill 0.3) (layers "F.Cu" "B.Cu") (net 14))
 (segment (start 230.285 43.375) (end 230.06 43.15) (width 0.2) (layer "B.Cu") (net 14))
 (segment (start 230.01 43.1) (end 230.035 43.125) (width 0.2) (layer "B.Cu") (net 14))
 (segment (start 230.06 43.1) (end 230.01 43.1) (width 0.2) (layer "B.Cu") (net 14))
 (segment (start 230.06 43.15) (end 230.06 43.1) (width 0.2) (layer "B.Cu") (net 14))
 (segment (start 235.035 43.375) (end 230.285 43.375) (width 0.2) (layer "B.Cu") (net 14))
 (segment (start 235.285 39.425) (end 235.385 39.325) (width 0.2) (layer "F.Cu") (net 8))
 (segment (start 229.41 40.625) (end 229.6235 40.4115) (width 0.2) (layer "F.Cu") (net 8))
 (segment (start 237.035 33.775) (end 237.035 37.675) (width 0.2) (layer "F.Cu") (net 8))
 (segment (start 237.035 37.675) (end 235.435 39.275) (width 0.2) (layer "F.Cu") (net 8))
 (segment (start 229.6235 40.4115) (end 231.8934 40.4115) (width 0.2) (layer "F.Cu") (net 8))
 (segment (start 235.435 39.275) (end 235.435 39.425) (width 0.2) (layer "F.Cu") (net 8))
 (segment (start 235.435 39.425) (end 235.285 39.425) (width 0.2) (layer "F.Cu") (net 8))
 (via (at 229.41 40.625) (size 0.6) (drill 0.3) (layers "F.Cu" "B.Cu") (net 8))
 (via (at 235.435 39.425) (size 0.6) (drill 0.3) (layers "F.Cu" "B.Cu") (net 8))
 (segment (start 229.41 40.625) (end 229.46 40.475) (width 0.2) (layer "B.Cu") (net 8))
 (segment (start 230.51 39.425) (end 229.41 40.625) (width 0.2) (layer "B.Cu") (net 8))
 (segment (start 235.435 39.425) (end 230.51 39.425) (width 0.2) (layer "B.Cu") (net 8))
 (segment (start 229.335 38.4) (end 229.8635 37.8715) (width 0.2) (layer "F.Cu") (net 9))
 (segment (start 237.035 31.235) (end 235.06 33.21) (width 0.2) (layer "F.Cu") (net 9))
 (segment (start 235.06 33.21) (end 235.06 36.925) (width 0.2) (layer "F.Cu") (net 9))
 (segment (start 235.61 37.475) (end 235.635 37.475) (width 0.2) (layer "F.Cu") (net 9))
 (segment (start 235.635 37.475) (end 235.635 37.5) (width 0.2) (layer "F.Cu") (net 9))
 (segment (start 235.635 37.5) (end 235.585 37.45) (width 0.2) (layer "F.Cu") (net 9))
 (segment (start 229.8635 37.8715) (end 231.8934 37.8715) (width 0.2) (layer "F.Cu") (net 9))
 (segment (start 235.06 36.925) (end 235.61 37.475) (width 0.2) (layer "F.Cu") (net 9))
 (via (at 235.635 37.475) (size 0.6) (drill 0.3) (layers "F.Cu" "B.Cu") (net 9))
 (via (at 229.335 38.4) (size 0.6) (drill 0.3) (layers "F.Cu" "B.Cu") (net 9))
 (segment (start 230.185 37.475) (end 229.335 38.4) (width 0.2) (layer "B.Cu") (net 9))
 (segment (start 235.635 37.475) (end 230.185 37.475) (width 0.2) (layer "B.Cu") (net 9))
 (segment (start 229.335 38.4) (end 229.385 38.275) (width 0.2) (layer "B.Cu") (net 9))
 (segment (start 231.72 65.6) (end 241.235 65.6) (width 0.2) (layer "F.Cu") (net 19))
 (segment (start 241.235 65.6) (end 242.92 63.915) (width 0.2) (layer "F.Cu") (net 19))
 (segment (start 225.57 71.75) (end 231.72 65.6) (width 0.2) (layer "F.Cu") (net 19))
 (segment (start 242.92 63.915) (end 242.92 60.85) (width 0.2) (layer "F.Cu") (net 19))
 (segment (start 230.16 48.325) (end 230.11 48.275) (width 0.2) (layer "F.Cu") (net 15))
 (segment (start 231.8934 35.3315) (end 230.5184 35.3315) (width 0.2) (layer "F.Cu") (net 15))
 (segment (start 228.71 37.1399) (end 228.71 46.875) (width 0.2) (layer "F.Cu") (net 15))
 (segment (start 233.185 66.625) (end 233.21 66.6) (width 0.2) (layer "F.Cu") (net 15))
 (segment (start 228.71 46.875) (end 230.135 48.3) (width 0.2) (layer "F.Cu") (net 15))
 (segment (start 233.21 66.69) (end 233.185 66.625) (width 0.2) (layer "F.Cu") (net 15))
 (segment (start 230.16 48.3) (end 230.16 48.325) (width 0.2) (layer "F.Cu") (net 15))
 (segment (start 230.135 48.3) (end 230.16 48.3) (width 0.2) (layer "F.Cu") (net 15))
 (segment (start 230.5184 35.3315) (end 228.71 37.1399) (width 0.2) (layer "F.Cu") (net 15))
 (segment (start 238.27 71.75) (end 233.21 66.69) (width 0.2) (layer "F.Cu") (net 15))
 (via (at 230.16 48.3) (size 0.6) (drill 0.3) (layers "F.Cu" "B.Cu") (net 15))
 (via (at 233.185 66.625) (size 0.6) (drill 0.3) (layers "F.Cu" "B.Cu") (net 15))
 (segment (start 233.91 50.675) (end 233.91 50.975) (width 0.2) (layer "B.Cu") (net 15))
 (segment (start 233.91 50.975) (end 233.91 52.375) (width 0.2) (layer "B.Cu") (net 15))
 (segment (start 233.385 50.15) (end 233.91 50.675) (width 0.2) (layer "B.Cu") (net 15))
 (segment (start 230.16 48.3) (end 231.535 48.3) (width 0.2) (layer "B.Cu") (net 15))
 (segment (start 233.91 52.375) (end 232.91 53.375) (width 0.2) (layer "B.Cu") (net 15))
 (segment (start 232.835 53.45) (end 232.86 53.425) (width 0.2) (layer "B.Cu") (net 15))
 (segment (start 232.91 53.45) (end 232.835 53.45) (width 0.2) (layer "B.Cu") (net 15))
 (segment (start 233.21 53.675) (end 233.21 66.625) (width 0.2) (layer "B.Cu") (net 15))
 (segment (start 231.535 48.3) (end 233.385 50.15) (width 0.2) (layer "B.Cu") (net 15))
 (segment (start 232.91 53.375) (end 232.91 53.45) (width 0.2) (layer "B.Cu") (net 15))
 (segment (start 232.91 53.375) (end 233.21 53.675) (width 0.2) (layer "B.Cu") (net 15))
 (segment (start 241.65 60.85) (end 241.65 56.635) (width 0.2) (layer "F.Cu") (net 20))
 (segment (start 241.65 56.635) (end 243.735 54.55) (width 0.2) (layer "F.Cu") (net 20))
 (segment (start 227.485 38.625) (end 220.86 38.625) (width 0.2) (layer "F.Cu") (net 16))
 (segment (start 235.73 71.75) (end 235.73 70.37) (width 0.2) (layer "F.Cu") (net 16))
 (segment (start 220.86 38.625) (end 220.735 38.5) (width 0.2) (layer "F.Cu") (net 16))
 (segment (start 235.73 70.37) (end 232.31 66.95) (width 0.2) (layer "F.Cu") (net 16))
 (segment (start 220.71 38.475) (end 220.71 38.475) (width 0.2) (layer "F.Cu") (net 16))
 (segment (start 220.735 38.5) (end 220.735 38.475) (width 0.2) (layer "F.Cu") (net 16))
 (segment (start 220.735 38.475) (end 220.71 38.475) (width 0.2) (layer "F.Cu") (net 16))
 (segment (start 232.31 66.95) (end 232.26 66.9) (width 0.2) (layer "F.Cu") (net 16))
 (via (at 227.485 38.625) (size 0.6) (drill 0.3) (layers "F.Cu" "B.Cu") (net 16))
 (via (at 232.31 66.95) (size 0.6) (drill 0.3) (layers "F.Cu" "B.Cu") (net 16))
 (via (at 220.735 38.475) (size 0.6) (drill 0.3) (layers "F.Cu" "B.Cu") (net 16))
 (segment (start 220.735 38.475) (end 220.735 31.005) (width 0.2) (layer "B.Cu") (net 16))
 (segment (start 227.485 38.625) (end 227.435 38.625) (width 0.2) (layer "B.Cu") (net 16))
 (segment (start 227.435 62.075) (end 227.485 38.625) (width 0.2) (layer "B.Cu") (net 16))
 (segment (start 220.735 31.005) (end 222.51 29.23) (width 0.2) (layer "B.Cu") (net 16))
 (segment (start 232.31 66.95) (end 227.435 62.075) (width 0.2) (layer "B.Cu") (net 16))
 (segment (start 229.06 69.375) (end 228.11 70.325) (width 0.2) (layer "F.Cu") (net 17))
 (segment (start 228.485 69.95) (end 228.485 69.95) (width 0.2) (layer "F.Cu") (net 17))
 (segment (start 228.485 69.875) (end 228.485 69.95) (width 0.2) (layer "F.Cu") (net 17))
 (segment (start 229.06 69.3) (end 229.06 69.375) (width 0.2) (layer "F.Cu") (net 17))
 (segment (start 228.11 70.325) (end 228.11 71.75) (width 0.2) (layer "F.Cu") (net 17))
 (via (at 229.06 69.3) (size 0.6) (drill 0.3) (layers "F.Cu" "B.Cu") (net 17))
 (segment (start 226.36 30.54) (end 225.05 29.23) (width 0.2) (layer "B.Cu") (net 17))
 (segment (start 229.06 69.325) (end 229.06 68.7) (width 0.2) (layer "B.Cu") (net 17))
 (segment (start 226.36 67.5) (end 226.36 30.54) (width 0.2) (layer "B.Cu") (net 17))
 (segment (start 227.86 67.5) (end 226.36 67.5) (width 0.2) (layer "B.Cu") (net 17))
 (segment (start 229.06 68.7) (end 227.86 67.5) (width 0.2) (layer "B.Cu") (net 17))
 (segment (start 216.485 48.761742) (end 218.171742 47.075) (width 0.2) (layer "F.Cu") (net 18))
 (segment (start 218.835 44.05) (end 218.81 44.05) (width 0.2) (layer "F.Cu") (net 18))
 (segment (start 216.41 68.65) (end 216.485 68.65) (width 0.2) (layer "F.Cu") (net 18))
 (segment (start 217.39 68.65) (end 216.41 68.65) (width 0.2) (layer "F.Cu") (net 18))
 (segment (start 218.81 47) (end 218.735 47.075) (width 0.2) (layer "F.Cu") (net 18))
 (segment (start 216.485 59.425) (end 216.485 48.761742) (width 0.2) (layer "F.Cu") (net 18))
 (segment (start 222.51 34.31) (end 218.81 38.01) (width 0.2) (layer "F.Cu") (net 18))
 (segment (start 220.49 71.75) (end 217.39 68.65) (width 0.2) (layer "F.Cu") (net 18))
 (segment (start 218.171742 47.075) (end 218.81 47) (width 0.2) (layer "F.Cu") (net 18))
 (segment (start 218.81 38.01) (end 218.835 44.05) (width 0.2) (layer "F.Cu") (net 18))
 (via (at 216.485 59.425) (size 0.6) (drill 0.3) (layers "F.Cu" "B.Cu") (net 18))
 (via (at 218.835 44.05) (size 0.6) (drill 0.3) (layers "F.Cu" "B.Cu") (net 18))
 (via (at 216.41 68.65) (size 0.6) (drill 0.3) (layers "F.Cu" "B.Cu") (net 18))
 (via (at 218.81 47) (size 0.6) (drill 0.3) (layers "F.Cu" "B.Cu") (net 18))
 (segment (start 216.46 59.4) (end 216.46 59.325) (width 0.2) (layer "B.Cu") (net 18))
 (segment (start 216.485 59.425) (end 216.46 59.4) (width 0.2) (layer "B.Cu") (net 18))
 (segment (start 218.835 46.975) (end 218.81 47) (width 0.2) (layer "B.Cu") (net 18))
 (segment (start 216.46 68.6) (end 216.46 59.45) (width 0.2) (layer "B.Cu") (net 18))
 (segment (start 216.41 68.65) (end 216.46 68.6) (width 0.2) (layer "B.Cu") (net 18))
 (segment (start 218.835 44.05) (end 218.835 46.975) (width 0.2) (layer "B.Cu") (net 18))
 (segment (start 216.46 59.45) (end 216.485 59.425) (width 0.2) (layer "B.Cu") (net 18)))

